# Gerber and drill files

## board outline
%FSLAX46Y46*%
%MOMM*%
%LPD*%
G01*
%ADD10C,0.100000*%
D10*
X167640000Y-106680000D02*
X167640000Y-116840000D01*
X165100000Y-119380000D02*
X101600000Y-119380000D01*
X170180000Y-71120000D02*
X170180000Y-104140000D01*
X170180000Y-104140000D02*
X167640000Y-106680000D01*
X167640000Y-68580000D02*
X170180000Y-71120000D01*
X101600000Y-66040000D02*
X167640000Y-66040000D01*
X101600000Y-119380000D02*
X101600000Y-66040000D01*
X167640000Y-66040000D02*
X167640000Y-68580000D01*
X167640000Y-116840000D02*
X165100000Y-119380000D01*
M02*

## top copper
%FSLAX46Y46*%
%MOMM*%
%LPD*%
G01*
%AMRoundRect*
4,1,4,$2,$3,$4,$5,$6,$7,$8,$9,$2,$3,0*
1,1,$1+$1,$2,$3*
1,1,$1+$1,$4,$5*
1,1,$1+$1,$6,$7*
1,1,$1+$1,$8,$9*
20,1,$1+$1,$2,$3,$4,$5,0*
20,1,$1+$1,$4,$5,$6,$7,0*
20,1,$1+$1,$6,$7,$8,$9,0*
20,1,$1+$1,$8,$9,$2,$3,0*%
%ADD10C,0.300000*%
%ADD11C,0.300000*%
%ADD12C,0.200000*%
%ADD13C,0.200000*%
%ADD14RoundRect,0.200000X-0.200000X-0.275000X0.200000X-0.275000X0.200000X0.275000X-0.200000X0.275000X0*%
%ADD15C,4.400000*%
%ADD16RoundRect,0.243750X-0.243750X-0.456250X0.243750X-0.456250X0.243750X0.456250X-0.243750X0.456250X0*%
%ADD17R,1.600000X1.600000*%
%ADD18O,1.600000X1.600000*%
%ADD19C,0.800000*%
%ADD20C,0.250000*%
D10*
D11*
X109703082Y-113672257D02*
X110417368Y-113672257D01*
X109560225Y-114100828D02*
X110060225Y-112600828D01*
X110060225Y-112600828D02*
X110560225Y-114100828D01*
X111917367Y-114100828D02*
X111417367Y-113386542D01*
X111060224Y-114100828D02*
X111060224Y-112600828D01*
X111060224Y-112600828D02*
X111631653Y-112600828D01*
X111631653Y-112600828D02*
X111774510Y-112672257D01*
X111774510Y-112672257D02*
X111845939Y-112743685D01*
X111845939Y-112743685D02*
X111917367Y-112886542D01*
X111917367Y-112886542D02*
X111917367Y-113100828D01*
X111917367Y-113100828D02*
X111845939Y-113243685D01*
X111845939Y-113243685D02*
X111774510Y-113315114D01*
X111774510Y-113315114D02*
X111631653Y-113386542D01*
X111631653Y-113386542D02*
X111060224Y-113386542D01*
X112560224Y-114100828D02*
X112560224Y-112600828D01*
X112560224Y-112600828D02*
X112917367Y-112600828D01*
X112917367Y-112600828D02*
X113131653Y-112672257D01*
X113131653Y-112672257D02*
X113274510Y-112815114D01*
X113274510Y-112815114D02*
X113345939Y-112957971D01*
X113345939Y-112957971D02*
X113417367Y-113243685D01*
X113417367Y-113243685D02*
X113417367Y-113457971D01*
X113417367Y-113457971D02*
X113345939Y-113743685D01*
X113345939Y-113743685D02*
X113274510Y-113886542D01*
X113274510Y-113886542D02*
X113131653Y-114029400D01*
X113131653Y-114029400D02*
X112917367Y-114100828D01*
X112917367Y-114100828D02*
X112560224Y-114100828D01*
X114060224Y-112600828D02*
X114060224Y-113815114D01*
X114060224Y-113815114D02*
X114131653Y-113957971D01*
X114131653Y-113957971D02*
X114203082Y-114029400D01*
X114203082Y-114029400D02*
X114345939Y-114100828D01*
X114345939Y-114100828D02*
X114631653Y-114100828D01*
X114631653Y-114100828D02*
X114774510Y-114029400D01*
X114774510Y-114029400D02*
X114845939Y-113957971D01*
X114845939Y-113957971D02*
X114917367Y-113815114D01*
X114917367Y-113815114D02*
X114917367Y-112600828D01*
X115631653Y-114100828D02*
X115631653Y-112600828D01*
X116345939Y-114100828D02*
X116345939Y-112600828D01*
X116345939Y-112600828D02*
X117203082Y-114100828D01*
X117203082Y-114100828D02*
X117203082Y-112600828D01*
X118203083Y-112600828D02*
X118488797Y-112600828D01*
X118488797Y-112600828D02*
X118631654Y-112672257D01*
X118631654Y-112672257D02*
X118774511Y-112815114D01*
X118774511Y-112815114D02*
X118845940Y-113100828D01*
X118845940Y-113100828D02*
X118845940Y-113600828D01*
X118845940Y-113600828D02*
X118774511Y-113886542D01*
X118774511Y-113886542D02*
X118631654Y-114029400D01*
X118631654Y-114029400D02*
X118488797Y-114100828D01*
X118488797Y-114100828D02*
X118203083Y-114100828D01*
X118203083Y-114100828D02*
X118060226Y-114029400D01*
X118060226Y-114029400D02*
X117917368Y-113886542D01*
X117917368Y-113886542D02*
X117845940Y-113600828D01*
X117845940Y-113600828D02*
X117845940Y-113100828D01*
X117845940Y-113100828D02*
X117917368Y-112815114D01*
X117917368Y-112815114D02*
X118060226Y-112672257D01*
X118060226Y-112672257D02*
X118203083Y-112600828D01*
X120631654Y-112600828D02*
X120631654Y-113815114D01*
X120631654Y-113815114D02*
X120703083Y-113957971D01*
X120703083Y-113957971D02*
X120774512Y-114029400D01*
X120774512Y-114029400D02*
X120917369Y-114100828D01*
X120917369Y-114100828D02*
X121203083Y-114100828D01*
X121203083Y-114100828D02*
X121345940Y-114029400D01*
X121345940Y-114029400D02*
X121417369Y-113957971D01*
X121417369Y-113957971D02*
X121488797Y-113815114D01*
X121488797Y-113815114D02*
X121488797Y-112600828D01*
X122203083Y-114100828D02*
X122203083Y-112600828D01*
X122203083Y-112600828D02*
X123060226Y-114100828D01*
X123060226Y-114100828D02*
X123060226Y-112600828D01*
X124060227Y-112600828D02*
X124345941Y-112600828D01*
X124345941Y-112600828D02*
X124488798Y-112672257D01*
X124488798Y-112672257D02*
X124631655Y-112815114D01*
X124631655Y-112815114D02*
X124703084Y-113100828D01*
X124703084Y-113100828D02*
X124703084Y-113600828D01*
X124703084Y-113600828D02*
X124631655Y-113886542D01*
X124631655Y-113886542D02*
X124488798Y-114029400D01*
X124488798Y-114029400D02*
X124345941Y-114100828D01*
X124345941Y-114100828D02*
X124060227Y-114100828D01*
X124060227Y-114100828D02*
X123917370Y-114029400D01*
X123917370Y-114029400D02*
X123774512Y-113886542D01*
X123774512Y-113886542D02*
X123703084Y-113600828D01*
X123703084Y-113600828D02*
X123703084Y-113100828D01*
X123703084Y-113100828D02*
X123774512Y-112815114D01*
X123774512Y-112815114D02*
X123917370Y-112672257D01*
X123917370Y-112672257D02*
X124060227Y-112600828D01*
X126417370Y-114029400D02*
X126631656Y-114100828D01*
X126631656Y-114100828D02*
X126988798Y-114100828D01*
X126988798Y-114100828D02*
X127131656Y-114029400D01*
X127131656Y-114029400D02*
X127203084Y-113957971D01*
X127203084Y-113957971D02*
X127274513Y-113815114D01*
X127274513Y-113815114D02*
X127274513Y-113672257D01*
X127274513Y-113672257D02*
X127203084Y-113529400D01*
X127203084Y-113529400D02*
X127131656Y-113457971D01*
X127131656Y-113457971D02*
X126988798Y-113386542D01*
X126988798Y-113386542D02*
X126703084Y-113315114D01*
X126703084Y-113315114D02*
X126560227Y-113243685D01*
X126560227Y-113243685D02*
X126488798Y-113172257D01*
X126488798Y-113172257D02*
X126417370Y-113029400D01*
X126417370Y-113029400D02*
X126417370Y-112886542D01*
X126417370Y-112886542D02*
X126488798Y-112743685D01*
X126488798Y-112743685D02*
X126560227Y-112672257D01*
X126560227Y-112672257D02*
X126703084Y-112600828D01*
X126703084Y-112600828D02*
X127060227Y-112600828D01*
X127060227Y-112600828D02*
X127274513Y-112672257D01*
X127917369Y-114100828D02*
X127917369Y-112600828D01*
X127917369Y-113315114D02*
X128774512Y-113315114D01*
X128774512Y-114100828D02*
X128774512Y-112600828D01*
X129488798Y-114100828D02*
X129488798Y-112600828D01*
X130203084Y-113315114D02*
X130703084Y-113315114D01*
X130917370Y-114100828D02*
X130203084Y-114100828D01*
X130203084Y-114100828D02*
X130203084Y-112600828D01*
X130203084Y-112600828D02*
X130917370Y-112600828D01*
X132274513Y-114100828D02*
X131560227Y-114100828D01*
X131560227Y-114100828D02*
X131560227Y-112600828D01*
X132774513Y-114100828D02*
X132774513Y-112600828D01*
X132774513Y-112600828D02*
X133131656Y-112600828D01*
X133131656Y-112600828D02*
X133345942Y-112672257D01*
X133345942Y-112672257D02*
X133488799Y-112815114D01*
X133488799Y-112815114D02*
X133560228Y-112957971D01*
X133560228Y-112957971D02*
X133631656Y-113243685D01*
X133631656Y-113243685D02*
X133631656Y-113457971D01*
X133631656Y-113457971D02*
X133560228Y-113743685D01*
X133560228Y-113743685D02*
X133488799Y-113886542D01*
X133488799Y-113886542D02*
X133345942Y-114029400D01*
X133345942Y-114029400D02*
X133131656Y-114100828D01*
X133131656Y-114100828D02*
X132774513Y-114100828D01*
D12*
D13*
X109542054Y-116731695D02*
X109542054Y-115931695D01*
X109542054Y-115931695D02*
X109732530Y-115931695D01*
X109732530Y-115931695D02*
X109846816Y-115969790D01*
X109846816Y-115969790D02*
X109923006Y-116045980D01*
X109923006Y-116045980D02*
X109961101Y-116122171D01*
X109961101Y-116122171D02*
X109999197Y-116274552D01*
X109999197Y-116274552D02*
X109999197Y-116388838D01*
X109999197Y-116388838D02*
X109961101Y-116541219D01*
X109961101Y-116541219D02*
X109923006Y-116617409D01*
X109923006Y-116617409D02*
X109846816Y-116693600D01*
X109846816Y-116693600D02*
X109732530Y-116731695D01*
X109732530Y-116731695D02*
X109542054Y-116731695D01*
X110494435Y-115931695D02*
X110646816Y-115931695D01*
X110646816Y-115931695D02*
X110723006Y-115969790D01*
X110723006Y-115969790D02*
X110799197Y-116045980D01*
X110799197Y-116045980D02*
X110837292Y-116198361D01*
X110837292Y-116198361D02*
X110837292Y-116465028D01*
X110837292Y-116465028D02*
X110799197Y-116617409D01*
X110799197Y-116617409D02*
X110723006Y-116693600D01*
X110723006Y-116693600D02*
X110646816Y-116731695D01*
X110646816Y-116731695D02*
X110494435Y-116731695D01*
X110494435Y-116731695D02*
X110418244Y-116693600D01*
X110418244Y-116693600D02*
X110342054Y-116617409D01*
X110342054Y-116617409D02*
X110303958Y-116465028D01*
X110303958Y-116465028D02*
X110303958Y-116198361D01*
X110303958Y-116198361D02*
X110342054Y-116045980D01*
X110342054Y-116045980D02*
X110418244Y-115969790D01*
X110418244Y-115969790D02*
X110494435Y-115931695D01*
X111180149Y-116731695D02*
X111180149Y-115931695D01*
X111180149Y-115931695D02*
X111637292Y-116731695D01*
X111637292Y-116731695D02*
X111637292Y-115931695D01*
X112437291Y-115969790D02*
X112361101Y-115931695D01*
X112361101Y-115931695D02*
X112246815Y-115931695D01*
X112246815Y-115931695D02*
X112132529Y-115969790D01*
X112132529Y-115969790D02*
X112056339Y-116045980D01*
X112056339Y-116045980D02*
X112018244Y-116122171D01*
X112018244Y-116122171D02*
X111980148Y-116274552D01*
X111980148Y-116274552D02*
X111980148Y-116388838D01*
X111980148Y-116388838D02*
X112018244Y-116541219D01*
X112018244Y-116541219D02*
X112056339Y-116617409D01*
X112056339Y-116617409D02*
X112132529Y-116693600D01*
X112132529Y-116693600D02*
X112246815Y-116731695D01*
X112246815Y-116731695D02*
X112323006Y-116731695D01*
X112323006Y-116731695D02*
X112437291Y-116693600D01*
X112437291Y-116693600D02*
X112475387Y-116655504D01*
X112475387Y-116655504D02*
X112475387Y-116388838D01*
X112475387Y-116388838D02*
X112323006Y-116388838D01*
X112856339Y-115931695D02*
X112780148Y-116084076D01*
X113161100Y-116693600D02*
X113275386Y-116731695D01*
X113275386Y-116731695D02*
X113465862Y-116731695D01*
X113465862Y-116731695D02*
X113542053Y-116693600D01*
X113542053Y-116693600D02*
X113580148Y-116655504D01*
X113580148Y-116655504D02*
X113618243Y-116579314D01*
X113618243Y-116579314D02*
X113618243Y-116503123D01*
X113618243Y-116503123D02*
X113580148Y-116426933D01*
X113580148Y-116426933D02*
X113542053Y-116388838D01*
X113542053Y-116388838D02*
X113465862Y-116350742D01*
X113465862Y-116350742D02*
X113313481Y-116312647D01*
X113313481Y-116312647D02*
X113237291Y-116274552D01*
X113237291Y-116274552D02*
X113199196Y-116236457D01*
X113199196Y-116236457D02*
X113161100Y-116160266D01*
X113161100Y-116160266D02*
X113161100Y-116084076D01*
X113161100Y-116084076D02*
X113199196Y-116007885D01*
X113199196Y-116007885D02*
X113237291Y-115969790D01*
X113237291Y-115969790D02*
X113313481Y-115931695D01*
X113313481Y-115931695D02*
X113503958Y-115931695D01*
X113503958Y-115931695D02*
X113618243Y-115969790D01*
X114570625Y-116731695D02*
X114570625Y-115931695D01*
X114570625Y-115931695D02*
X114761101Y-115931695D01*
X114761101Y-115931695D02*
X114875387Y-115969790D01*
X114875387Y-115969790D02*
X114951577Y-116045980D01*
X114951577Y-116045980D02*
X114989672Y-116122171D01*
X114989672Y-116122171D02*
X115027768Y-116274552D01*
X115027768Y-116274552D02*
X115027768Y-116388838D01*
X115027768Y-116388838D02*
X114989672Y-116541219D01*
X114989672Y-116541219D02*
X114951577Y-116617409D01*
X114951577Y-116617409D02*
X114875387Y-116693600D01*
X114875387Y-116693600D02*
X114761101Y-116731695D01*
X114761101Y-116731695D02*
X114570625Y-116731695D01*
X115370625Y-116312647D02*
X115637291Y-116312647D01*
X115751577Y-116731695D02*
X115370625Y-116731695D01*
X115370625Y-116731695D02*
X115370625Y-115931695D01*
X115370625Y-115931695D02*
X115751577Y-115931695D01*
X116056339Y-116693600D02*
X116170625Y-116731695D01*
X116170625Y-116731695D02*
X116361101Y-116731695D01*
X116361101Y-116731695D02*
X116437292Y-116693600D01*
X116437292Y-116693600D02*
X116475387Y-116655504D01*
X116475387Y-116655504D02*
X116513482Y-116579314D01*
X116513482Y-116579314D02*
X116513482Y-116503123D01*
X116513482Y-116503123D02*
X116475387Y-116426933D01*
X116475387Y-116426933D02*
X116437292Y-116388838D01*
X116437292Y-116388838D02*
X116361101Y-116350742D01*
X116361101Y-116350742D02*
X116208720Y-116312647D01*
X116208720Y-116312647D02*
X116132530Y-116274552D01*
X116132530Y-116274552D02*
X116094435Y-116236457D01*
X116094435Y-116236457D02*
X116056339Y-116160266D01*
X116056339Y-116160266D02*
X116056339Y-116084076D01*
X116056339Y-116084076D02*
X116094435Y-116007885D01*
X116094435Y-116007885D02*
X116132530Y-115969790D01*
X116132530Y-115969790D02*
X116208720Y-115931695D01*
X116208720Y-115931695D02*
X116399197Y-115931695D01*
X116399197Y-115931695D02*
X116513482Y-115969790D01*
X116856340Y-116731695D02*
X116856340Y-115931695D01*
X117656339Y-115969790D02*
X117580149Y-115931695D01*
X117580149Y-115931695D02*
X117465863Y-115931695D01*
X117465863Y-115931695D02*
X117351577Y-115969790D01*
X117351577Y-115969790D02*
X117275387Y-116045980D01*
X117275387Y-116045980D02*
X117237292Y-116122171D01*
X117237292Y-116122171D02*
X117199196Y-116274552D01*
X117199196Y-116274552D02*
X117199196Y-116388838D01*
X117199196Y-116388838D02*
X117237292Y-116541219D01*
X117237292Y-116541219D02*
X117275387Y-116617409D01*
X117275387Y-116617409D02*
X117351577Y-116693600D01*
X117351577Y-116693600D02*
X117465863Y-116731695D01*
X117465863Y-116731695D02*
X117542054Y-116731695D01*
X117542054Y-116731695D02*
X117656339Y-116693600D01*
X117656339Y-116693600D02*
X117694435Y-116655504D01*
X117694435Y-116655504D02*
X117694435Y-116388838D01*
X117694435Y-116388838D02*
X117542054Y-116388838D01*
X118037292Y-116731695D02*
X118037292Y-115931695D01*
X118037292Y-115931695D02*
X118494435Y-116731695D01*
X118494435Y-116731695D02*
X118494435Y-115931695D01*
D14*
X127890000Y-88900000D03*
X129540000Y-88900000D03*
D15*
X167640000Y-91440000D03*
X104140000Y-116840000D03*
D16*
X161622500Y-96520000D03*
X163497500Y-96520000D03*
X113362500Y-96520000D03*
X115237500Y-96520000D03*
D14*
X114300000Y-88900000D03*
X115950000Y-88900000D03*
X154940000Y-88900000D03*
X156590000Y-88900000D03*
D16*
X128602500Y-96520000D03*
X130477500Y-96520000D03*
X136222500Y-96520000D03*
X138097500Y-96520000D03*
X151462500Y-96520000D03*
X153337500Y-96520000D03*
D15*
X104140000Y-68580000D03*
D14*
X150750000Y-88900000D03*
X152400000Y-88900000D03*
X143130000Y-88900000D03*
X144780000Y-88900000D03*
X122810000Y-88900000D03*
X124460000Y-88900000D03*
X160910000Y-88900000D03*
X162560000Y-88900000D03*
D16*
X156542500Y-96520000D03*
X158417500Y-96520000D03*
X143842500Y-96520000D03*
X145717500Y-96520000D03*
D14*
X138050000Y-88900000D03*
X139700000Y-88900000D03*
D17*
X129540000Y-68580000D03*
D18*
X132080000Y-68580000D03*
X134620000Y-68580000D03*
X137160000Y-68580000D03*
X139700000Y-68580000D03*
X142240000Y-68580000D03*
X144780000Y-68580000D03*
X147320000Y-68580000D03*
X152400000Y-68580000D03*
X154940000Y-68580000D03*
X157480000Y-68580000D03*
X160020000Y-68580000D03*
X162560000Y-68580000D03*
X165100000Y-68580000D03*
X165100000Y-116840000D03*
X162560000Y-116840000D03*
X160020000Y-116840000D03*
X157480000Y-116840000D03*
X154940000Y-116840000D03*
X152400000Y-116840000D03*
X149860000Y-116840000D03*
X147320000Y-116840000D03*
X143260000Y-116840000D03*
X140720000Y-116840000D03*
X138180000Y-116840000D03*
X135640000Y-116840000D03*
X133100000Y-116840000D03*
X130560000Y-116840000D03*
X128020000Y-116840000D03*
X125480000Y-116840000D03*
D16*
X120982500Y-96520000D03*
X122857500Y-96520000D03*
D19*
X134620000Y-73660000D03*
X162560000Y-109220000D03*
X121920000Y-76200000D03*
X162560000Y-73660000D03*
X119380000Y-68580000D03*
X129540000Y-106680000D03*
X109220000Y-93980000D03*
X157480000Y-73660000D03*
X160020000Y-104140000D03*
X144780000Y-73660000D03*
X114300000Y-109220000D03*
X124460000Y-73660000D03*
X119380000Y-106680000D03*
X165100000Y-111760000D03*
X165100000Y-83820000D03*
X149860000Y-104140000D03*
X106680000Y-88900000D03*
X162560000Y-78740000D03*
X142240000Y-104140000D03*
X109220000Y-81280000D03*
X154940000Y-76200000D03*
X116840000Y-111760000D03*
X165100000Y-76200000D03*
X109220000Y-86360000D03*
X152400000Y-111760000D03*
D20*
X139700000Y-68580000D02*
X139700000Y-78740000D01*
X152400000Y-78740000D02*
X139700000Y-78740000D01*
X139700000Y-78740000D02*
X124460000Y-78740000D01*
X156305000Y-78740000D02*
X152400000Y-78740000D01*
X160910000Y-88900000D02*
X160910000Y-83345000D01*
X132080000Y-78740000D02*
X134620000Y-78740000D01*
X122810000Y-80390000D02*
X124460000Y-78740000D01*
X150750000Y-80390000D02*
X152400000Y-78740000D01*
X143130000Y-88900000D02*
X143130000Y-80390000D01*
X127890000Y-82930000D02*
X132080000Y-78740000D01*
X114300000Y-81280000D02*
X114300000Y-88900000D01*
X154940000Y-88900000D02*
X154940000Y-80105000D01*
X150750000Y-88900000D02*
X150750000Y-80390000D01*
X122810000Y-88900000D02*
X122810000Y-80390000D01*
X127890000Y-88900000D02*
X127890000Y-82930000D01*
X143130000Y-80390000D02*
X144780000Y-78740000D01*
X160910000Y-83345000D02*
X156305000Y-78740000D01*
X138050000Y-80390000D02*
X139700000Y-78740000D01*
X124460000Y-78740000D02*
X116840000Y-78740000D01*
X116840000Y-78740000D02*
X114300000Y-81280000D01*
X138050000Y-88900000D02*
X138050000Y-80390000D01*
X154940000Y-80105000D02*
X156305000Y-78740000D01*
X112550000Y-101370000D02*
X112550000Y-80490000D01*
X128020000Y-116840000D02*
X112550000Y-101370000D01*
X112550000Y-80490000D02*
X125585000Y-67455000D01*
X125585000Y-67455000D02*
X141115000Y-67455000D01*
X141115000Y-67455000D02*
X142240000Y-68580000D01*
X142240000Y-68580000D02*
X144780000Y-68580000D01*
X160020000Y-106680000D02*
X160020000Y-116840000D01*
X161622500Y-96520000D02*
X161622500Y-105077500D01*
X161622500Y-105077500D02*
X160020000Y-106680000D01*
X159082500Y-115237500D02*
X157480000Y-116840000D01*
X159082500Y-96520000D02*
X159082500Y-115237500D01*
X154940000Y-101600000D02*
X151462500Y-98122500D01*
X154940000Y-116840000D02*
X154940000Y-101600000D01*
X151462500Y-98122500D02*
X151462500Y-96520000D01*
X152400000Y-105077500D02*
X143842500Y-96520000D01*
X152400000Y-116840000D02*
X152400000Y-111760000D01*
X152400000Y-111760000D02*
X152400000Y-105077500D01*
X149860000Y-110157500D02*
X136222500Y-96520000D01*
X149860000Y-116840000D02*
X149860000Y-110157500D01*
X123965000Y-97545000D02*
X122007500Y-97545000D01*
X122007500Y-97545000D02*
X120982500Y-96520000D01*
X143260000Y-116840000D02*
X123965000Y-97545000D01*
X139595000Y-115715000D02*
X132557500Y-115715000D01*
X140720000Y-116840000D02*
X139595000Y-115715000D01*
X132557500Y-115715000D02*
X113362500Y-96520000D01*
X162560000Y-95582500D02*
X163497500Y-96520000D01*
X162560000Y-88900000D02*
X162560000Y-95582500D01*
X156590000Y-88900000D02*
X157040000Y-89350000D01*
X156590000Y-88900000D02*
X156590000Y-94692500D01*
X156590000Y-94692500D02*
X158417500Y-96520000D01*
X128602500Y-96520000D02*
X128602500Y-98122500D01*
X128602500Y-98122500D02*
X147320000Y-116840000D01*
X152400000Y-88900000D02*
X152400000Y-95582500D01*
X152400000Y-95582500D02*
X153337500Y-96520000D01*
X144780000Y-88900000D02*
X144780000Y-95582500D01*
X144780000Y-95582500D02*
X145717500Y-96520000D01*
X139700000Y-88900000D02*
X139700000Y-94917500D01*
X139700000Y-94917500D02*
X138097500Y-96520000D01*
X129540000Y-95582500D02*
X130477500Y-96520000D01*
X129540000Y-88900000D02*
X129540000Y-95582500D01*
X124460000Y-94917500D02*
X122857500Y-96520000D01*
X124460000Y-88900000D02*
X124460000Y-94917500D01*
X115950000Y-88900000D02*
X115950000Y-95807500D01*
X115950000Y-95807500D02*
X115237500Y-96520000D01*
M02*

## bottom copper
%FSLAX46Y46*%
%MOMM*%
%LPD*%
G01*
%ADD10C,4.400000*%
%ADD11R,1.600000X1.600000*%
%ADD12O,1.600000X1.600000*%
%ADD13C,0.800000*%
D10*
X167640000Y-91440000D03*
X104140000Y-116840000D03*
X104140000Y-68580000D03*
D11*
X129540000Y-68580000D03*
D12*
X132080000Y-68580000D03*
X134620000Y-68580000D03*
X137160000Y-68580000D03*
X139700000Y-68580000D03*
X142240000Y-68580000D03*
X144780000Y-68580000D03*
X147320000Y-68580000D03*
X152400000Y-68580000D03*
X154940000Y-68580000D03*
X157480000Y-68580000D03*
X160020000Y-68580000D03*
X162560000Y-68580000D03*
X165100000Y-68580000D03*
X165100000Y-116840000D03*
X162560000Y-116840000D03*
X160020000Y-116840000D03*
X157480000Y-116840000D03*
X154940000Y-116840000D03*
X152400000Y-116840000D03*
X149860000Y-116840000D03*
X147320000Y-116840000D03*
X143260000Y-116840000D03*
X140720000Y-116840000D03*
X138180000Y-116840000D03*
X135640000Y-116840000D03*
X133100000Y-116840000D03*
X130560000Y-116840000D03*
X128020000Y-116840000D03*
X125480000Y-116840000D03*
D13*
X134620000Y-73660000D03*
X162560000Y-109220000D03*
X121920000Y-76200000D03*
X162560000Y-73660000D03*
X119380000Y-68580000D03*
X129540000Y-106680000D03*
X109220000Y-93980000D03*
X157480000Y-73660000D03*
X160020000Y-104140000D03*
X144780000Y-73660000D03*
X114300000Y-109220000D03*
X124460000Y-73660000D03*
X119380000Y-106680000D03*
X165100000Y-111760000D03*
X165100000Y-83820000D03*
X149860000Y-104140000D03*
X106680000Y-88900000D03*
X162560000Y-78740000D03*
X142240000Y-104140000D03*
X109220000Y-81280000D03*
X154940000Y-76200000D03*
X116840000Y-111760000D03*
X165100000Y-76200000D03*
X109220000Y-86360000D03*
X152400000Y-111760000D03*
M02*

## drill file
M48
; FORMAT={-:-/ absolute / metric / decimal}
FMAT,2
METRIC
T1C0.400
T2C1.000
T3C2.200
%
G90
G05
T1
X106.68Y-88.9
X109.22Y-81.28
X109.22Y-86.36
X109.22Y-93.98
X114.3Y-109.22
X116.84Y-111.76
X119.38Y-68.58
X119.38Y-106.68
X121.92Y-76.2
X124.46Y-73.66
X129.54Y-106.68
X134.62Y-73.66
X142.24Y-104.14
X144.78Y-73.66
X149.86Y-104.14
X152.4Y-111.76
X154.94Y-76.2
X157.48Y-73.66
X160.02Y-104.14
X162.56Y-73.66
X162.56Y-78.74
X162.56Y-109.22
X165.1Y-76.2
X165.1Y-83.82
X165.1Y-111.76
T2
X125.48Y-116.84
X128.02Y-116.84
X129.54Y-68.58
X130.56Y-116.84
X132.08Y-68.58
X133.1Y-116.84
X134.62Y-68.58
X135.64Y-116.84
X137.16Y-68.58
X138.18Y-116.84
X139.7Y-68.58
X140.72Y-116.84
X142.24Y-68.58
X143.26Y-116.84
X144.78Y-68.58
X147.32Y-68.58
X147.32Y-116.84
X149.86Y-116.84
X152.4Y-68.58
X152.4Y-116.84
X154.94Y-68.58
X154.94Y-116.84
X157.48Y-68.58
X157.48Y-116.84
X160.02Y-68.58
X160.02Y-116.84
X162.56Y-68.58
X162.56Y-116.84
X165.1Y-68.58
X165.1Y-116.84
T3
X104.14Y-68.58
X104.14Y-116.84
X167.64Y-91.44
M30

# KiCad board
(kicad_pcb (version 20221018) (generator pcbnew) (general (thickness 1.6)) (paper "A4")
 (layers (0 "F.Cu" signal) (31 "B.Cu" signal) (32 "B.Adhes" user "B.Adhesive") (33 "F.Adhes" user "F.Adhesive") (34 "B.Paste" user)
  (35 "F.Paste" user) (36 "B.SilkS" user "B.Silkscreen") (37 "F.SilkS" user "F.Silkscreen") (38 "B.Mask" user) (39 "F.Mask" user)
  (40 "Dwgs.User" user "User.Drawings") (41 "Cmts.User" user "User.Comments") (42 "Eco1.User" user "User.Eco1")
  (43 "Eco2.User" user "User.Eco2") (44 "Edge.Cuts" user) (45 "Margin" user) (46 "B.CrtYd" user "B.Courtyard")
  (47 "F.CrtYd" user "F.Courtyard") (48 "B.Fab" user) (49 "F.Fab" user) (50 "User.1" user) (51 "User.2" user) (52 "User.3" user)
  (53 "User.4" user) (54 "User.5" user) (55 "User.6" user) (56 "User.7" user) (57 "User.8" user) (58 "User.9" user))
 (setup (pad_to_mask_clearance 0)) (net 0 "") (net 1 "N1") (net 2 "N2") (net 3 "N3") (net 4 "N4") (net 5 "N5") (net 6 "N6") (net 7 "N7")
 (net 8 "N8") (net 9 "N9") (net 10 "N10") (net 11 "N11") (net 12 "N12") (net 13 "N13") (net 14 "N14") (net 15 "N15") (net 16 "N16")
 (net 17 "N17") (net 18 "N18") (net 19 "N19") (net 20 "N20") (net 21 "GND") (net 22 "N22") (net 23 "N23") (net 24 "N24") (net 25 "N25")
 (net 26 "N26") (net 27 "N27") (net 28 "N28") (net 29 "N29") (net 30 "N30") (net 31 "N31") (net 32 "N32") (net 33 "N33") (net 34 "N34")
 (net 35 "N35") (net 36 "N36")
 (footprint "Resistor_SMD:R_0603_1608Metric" (layer "F.Cu") (at 128.715 88.9)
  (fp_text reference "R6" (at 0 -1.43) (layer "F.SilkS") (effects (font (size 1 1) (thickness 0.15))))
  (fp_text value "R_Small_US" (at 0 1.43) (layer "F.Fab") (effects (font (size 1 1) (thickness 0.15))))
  (pad "1" smd roundrect (at -0.825 0) (size 0.8 0.95) (layers "F.Cu" "F.Paste" "F.Mask") (roundrect_rratio 0.25) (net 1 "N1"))
  (pad "2" smd roundrect (at 0.825 0) (size 0.8 0.95) (layers "F.Cu" "F.Paste" "F.Mask") (roundrect_rratio 0.25) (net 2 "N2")))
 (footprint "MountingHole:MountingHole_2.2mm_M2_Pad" (layer "F.Cu") (at 167.64 91.44)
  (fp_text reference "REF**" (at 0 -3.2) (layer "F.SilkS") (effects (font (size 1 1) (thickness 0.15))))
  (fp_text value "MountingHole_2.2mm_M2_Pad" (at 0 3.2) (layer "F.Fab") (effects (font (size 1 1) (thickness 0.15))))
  (pad "1" thru_hole circle (at 0 0) (size 4.4 4.4) (drill 2.2) (layers "*.Cu" "*.Mask")))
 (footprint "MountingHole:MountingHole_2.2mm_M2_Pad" (layer "F.Cu") (at 104.14 116.84)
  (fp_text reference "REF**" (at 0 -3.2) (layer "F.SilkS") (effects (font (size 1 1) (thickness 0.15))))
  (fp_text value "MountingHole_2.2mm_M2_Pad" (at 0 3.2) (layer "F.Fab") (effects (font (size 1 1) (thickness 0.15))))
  (pad "1" thru_hole circle (at 0 0) (size 4.4 4.4) (drill 2.2) (layers "*.Cu" "*.Mask")))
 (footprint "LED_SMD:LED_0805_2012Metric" (layer "F.Cu") (at 162.56 96.52)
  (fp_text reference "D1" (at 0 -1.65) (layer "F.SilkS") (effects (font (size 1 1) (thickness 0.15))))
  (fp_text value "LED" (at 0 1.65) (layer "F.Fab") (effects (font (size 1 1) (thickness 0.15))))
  (pad "1" smd roundrect (at -0.9375 0) (size 0.975 1.4) (layers "F.Cu" "F.Paste" "F.Mask") (roundrect_rratio 0.25) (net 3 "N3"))
  (pad "2" smd roundrect (at 0.9375 0) (size 0.975 1.4) (layers "F.Cu" "F.Paste" "F.Mask") (roundrect_rratio 0.25) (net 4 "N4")))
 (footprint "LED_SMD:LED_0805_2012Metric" (layer "F.Cu") (at 114.3 96.52)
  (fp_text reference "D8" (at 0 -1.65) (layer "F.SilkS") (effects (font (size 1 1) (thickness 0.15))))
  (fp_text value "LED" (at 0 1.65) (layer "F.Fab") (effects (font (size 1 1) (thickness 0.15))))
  (pad "1" smd roundrect (at -0.9375 0) (size 0.975 1.4) (layers "F.Cu" "F.Paste" "F.Mask") (roundrect_rratio 0.25) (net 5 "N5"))
  (pad "2" smd roundrect (at 0.9375 0) (size 0.975 1.4) (layers "F.Cu" "F.Paste" "F.Mask") (roundrect_rratio 0.25) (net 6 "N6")))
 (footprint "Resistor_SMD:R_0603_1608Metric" (layer "F.Cu") (at 115.125 88.9)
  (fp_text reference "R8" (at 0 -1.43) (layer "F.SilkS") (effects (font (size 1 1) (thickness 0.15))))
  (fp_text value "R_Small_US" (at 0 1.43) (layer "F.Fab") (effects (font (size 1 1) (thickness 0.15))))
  (pad "1" smd roundrect (at -0.825 0) (size 0.8 0.95) (layers "F.Cu" "F.Paste" "F.Mask") (roundrect_rratio 0.25) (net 1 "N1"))
  (pad "2" smd roundrect (at 0.825 0) (size 0.8 0.95) (layers "F.Cu" "F.Paste" "F.Mask") (roundrect_rratio 0.25) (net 6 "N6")))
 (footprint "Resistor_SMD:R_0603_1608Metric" (layer "F.Cu") (at 155.765 88.9)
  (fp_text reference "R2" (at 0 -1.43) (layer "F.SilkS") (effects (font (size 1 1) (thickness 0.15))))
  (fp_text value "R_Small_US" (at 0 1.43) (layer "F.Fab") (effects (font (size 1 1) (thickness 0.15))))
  (pad "1" smd roundrect (at -0.825 0) (size 0.8 0.95) (layers "F.Cu" "F.Paste" "F.Mask") (roundrect_rratio 0.25) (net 1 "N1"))
  (pad "2" smd roundrect (at 0.825 0) (size 0.8 0.95) (layers "F.Cu" "F.Paste" "F.Mask") (roundrect_rratio 0.25) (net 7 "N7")))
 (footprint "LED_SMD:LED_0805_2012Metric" (layer "F.Cu") (at 129.54 96.52)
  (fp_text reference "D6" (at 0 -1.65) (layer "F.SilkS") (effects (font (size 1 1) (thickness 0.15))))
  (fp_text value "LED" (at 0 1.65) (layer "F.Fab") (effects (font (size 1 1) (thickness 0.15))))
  (pad "1" smd roundrect (at -0.9375 0) (size 0.975 1.4) (layers "F.Cu" "F.Paste" "F.Mask") (roundrect_rratio 0.25) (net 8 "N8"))
  (pad "2" smd roundrect (at 0.9375 0) (size 0.975 1.4) (layers "F.Cu" "F.Paste" "F.Mask") (roundrect_rratio 0.25) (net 2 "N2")))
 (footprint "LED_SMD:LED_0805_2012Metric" (layer "F.Cu") (at 137.16 96.52)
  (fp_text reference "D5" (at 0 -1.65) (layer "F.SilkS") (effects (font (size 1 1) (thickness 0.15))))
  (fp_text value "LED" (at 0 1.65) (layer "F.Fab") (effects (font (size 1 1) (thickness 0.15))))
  (pad "1" smd roundrect (at -0.9375 0) (size 0.975 1.4) (layers "F.Cu" "F.Paste" "F.Mask") (roundrect_rratio 0.25) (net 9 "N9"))
  (pad "2" smd roundrect (at 0.9375 0) (size 0.975 1.4) (layers "F.Cu" "F.Paste" "F.Mask") (roundrect_rratio 0.25) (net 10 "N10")))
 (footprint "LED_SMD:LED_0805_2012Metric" (layer "F.Cu") (at 152.4 96.52)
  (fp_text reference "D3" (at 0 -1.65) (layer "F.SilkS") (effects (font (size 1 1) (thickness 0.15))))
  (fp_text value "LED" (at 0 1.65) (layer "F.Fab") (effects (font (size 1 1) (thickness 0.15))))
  (pad "1" smd roundrect (at -0.9375 0) (size 0.975 1.4) (layers "F.Cu" "F.Paste" "F.Mask") (roundrect_rratio 0.25) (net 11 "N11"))
  (pad "2" smd roundrect (at 0.9375 0) (size 0.975 1.4) (layers "F.Cu" "F.Paste" "F.Mask") (roundrect_rratio 0.25) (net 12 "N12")))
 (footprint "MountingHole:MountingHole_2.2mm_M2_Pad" (layer "F.Cu") (at 104.14 68.58)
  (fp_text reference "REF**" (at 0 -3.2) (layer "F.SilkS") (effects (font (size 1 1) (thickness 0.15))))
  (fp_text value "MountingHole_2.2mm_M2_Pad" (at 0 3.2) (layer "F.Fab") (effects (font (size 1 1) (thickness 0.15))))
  (pad "1" thru_hole circle (at 0 0) (size 4.4 4.4) (drill 2.2) (layers "*.Cu" "*.Mask")))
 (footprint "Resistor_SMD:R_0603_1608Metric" (layer "F.Cu") (at 151.575 88.9)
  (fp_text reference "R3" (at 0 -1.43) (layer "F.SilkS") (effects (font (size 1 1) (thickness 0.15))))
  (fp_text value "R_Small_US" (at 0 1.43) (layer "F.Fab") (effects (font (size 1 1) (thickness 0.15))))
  (pad "1" smd roundrect (at -0.825 0) (size 0.8 0.95) (layers "F.Cu" "F.Paste" "F.Mask") (roundrect_rratio 0.25) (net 1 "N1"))
  (pad "2" smd roundrect (at 0.825 0) (size 0.8 0.95) (layers "F.Cu" "F.Paste" "F.Mask") (roundrect_rratio 0.25) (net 12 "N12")))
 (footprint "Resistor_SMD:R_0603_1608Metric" (layer "F.Cu") (at 143.955 88.9)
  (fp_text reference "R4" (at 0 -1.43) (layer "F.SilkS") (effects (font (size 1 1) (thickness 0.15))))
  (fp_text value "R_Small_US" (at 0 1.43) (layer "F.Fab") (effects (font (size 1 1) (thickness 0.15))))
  (pad "1" smd roundrect (at -0.825 0) (size 0.8 0.95) (layers "F.Cu" "F.Paste" "F.Mask") (roundrect_rratio 0.25) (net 1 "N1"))
  (pad "2" smd roundrect (at 0.825 0) (size 0.8 0.95) (layers "F.Cu" "F.Paste" "F.Mask") (roundrect_rratio 0.25) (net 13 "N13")))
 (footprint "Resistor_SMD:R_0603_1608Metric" (layer "F.Cu") (at 123.635 88.9)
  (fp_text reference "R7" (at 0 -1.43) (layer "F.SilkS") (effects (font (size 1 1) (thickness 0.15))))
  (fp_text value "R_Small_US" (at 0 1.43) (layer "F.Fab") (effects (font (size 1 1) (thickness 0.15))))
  (pad "1" smd roundrect (at -0.825 0) (size 0.8 0.95) (layers "F.Cu" "F.Paste" "F.Mask") (roundrect_rratio 0.25) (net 1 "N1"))
  (pad "2" smd roundrect (at 0.825 0) (size 0.8 0.95) (layers "F.Cu" "F.Paste" "F.Mask") (roundrect_rratio 0.25) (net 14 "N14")))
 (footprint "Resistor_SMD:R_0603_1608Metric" (layer "F.Cu") (at 161.735 88.9)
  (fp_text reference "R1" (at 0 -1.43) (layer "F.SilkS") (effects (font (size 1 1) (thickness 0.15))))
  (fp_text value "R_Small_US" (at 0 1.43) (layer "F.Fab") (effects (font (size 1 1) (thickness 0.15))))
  (pad "1" smd roundrect (at -0.825 0) (size 0.8 0.95) (layers "F.Cu" "F.Paste" "F.Mask") (roundrect_rratio 0.25) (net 1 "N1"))
  (pad "2" smd roundrect (at 0.825 0) (size 0.8 0.95) (layers "F.Cu" "F.Paste" "F.Mask") (roundrect_rratio 0.25) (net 4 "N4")))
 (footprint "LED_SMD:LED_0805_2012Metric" (layer "F.Cu") (at 157.48 96.52)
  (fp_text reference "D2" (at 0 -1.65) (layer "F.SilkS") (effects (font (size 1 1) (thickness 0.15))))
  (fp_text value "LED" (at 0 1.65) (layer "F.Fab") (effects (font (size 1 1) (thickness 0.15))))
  (pad "1" smd roundrect (at -0.9375 0) (size 0.975 1.4) (layers "F.Cu" "F.Paste" "F.Mask") (roundrect_rratio 0.25) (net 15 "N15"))
  (pad "2" smd roundrect (at 0.9375 0) (size 0.975 1.4) (layers "F.Cu" "F.Paste" "F.Mask") (roundrect_rratio 0.25) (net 7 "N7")))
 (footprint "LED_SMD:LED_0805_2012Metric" (layer "F.Cu") (at 144.78 96.52)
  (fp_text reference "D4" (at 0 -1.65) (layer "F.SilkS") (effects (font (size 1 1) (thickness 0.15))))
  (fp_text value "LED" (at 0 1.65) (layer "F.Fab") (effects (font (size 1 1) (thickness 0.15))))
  (pad "1" smd roundrect (at -0.9375 0) (size 0.975 1.4) (layers "F.Cu" "F.Paste" "F.Mask") (roundrect_rratio 0.25) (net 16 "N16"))
  (pad "2" smd roundrect (at 0.9375 0) (size 0.975 1.4) (layers "F.Cu" "F.Paste" "F.Mask") (roundrect_rratio 0.25) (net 13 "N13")))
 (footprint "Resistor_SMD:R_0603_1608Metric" (layer "F.Cu") (at 138.875 88.9)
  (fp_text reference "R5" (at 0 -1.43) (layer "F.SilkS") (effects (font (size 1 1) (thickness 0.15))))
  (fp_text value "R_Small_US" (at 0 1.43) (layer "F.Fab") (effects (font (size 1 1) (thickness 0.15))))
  (pad "1" smd roundrect (at -0.825 0) (size 0.8 0.95) (layers "F.Cu" "F.Paste" "F.Mask") (roundrect_rratio 0.25) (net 1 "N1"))
  (pad "2" smd roundrect (at 0.825 0) (size 0.8 0.95) (layers "F.Cu" "F.Paste" "F.Mask") (roundrect_rratio 0.25) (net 10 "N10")))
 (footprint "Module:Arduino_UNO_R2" (layer "F.Cu") (at 129.54 68.58)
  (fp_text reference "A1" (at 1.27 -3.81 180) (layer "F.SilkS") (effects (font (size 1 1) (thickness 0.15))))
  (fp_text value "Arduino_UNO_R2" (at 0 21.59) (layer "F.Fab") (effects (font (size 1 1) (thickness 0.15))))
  (pad "1" thru_hole rect (at 0 0 90) (size 1.6 1.6) (drill 1) (layers "*.Cu" "*.Mask") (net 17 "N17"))
  (pad "2" thru_hole oval (at 2.54 0 90) (size 1.6 1.6) (drill 1) (layers "*.Cu" "*.Mask") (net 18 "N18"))
  (pad "3" thru_hole oval (at 5.08 0 90) (size 1.6 1.6) (drill 1) (layers "*.Cu" "*.Mask") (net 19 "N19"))
  (pad "4" thru_hole oval (at 7.62 0 90) (size 1.6 1.6) (drill 1) (layers "*.Cu" "*.Mask") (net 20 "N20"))
  (pad "5" thru_hole oval (at 10.16 0 90) (size 1.6 1.6) (drill 1) (layers "*.Cu" "*.Mask") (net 1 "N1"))
  (pad "6" thru_hole oval (at 12.7 0 90) (size 1.6 1.6) (drill 1) (layers "*.Cu" "*.Mask") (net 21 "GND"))
  (pad "7" thru_hole oval (at 15.24 0 90) (size 1.6 1.6) (drill 1) (layers "*.Cu" "*.Mask") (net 21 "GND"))
  (pad "8" thru_hole oval (at 17.78 0 90) (size 1.6 1.6) (drill 1) (layers "*.Cu" "*.Mask") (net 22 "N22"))
  (pad "9" thru_hole oval (at 22.86 0 90) (size 1.6 1.6) (drill 1) (layers "*.Cu" "*.Mask") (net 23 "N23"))
  (pad "10" thru_hole oval (at 25.4 0 90) (size 1.6 1.6) (drill 1) (layers "*.Cu" "*.Mask") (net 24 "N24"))
  (pad "11" thru_hole oval (at 27.94 0 90) (size 1.6 1.6) (drill 1) (layers "*.Cu" "*.Mask") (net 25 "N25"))
  (pad "12" thru_hole oval (at 30.48 0 90) (size 1.6 1.6) (drill 1) (layers "*.Cu" "*.Mask") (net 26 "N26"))
  (pad "13" thru_hole oval (at 33.02 0 90) (size 1.6 1.6) (drill 1) (layers "*.Cu" "*.Mask") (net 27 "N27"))
  (pad "14" thru_hole oval (at 35.56 0 90) (size 1.6 1.6) (drill 1) (layers "*.Cu" "*.Mask") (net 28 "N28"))
  (pad "15" thru_hole oval (at 35.56 48.26 90) (size 1.6 1.6) (drill 1) (layers "*.Cu" "*.Mask") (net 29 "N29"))
  (pad "16" thru_hole oval (at 33.02 48.26 90) (size 1.6 1.6) (drill 1) (layers "*.Cu" "*.Mask") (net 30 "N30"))
  (pad "17" thru_hole oval (at 30.48 48.26 90) (size 1.6 1.6) (drill 1) (layers "*.Cu" "*.Mask") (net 3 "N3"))
  (pad "18" thru_hole oval (at 27.94 48.26 90) (size 1.6 1.6) (drill 1) (layers "*.Cu" "*.Mask") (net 15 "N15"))
  (pad "19" thru_hole oval (at 25.4 48.26 90) (size 1.6 1.6) (drill 1) (layers "*.Cu" "*.Mask") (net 11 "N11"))
  (pad "20" thru_hole oval (at 22.86 48.26 90) (size 1.6 1.6) (drill 1) (layers "*.Cu" "*.Mask") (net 16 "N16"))
  (pad "21" thru_hole oval (at 20.32 48.26 90) (size 1.6 1.6) (drill 1) (layers "*.Cu" "*.Mask") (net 9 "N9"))
  (pad "22" thru_hole oval (at 17.78 48.26 90) (size 1.6 1.6) (drill 1) (layers "*.Cu" "*.Mask") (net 8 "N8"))
  (pad "23" thru_hole oval (at 13.72 48.26 90) (size 1.6 1.6) (drill 1) (layers "*.Cu" "*.Mask") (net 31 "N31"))
  (pad "24" thru_hole oval (at 11.18 48.26 90) (size 1.6 1.6) (drill 1) (layers "*.Cu" "*.Mask") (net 5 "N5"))
  (pad "25" thru_hole oval (at 8.64 48.26 90) (size 1.6 1.6) (drill 1) (layers "*.Cu" "*.Mask") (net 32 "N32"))
  (pad "26" thru_hole oval (at 6.1 48.26 90) (size 1.6 1.6) (drill 1) (layers "*.Cu" "*.Mask") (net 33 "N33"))
  (pad "27" thru_hole oval (at 3.56 48.26 90) (size 1.6 1.6) (drill 1) (layers "*.Cu" "*.Mask") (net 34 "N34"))
  (pad "28" thru_hole oval (at 1.02 48.26 90) (size 1.6 1.6) (drill 1) (layers "*.Cu" "*.Mask") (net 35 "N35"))
  (pad "29" thru_hole oval (at -1.52 48.26 90) (size 1.6 1.6) (drill 1) (layers "*.Cu" "*.Mask") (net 21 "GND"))
  (pad "30" thru_hole oval (at -4.06 48.26 90) (size 1.6 1.6) (drill 1) (layers "*.Cu" "*.Mask") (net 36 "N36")))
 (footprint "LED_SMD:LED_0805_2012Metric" (layer "F.Cu") (at 121.92 96.52)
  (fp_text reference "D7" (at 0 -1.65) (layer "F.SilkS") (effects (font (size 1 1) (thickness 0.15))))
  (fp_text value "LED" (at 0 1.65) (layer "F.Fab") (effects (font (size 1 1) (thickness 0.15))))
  (pad "1" smd roundrect (at -0.9375 0) (size 0.975 1.4) (layers "F.Cu" "F.Paste" "F.Mask") (roundrect_rratio 0.25) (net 31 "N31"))
  (pad "2" smd roundrect (at 0.9375 0) (size 0.975 1.4) (layers "F.Cu" "F.Paste" "F.Mask") (roundrect_rratio 0.25) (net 14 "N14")))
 (gr_line (start 167.64 106.68) (end 167.64 116.84) (stroke (width 0.1) (type default)) (layer "Edge.Cuts"))
 (gr_line (start 165.1 119.38) (end 101.6 119.38) (stroke (width 0.1) (type default)) (layer "Edge.Cuts"))
 (gr_line (start 170.18 71.12) (end 170.18 104.14) (stroke (width 0.1) (type default)) (layer "Edge.Cuts"))
 (gr_line (start 170.18 104.14) (end 167.64 106.68) (stroke (width 0.1) (type default)) (layer "Edge.Cuts"))
 (gr_line (start 167.64 68.58) (end 170.18 71.12) (stroke (width 0.1) (type default)) (layer "Edge.Cuts"))
 (gr_line (start 101.6 66.04) (end 167.64 66.04) (stroke (width 0.1) (type default)) (layer "Edge.Cuts"))
 (gr_line (start 101.6 119.38) (end 101.6 66.04) (stroke (width 0.1) (type default)) (layer "Edge.Cuts"))
 (gr_line (start 167.64 66.04) (end 167.64 68.58) (stroke (width 0.1) (type default)) (layer "Edge.Cuts"))
 (gr_line (start 167.64 116.84) (end 165.1 119.38) (stroke (width 0.1) (type default)) (layer "Edge.Cuts"))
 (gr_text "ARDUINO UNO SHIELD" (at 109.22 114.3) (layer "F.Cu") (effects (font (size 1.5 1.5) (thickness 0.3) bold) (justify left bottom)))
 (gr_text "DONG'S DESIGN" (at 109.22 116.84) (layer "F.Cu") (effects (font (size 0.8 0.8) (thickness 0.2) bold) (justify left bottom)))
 (via (at 134.62 73.66) (size 0.8) (drill 0.4) (layers "F.Cu" "B.Cu") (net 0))
 (via (at 162.56 109.22) (size 0.8) (drill 0.4) (layers "F.Cu" "B.Cu") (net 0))
 (via (at 121.92 76.2) (size 0.8) (drill 0.4) (layers "F.Cu" "B.Cu") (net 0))
 (via (at 162.56 73.66) (size 0.8) (drill 0.4) (layers "F.Cu" "B.Cu") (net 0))
 (via (at 119.38 68.58) (size 0.8) (drill 0.4) (layers "F.Cu" "B.Cu") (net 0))
 (via (at 129.54 106.68) (size 0.8) (drill 0.4) (layers "F.Cu" "B.Cu") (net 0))
 (via (at 109.22 93.98) (size 0.8) (drill 0.4) (layers "F.Cu" "B.Cu") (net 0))
 (via (at 157.48 73.66) (size 0.8) (drill 0.4) (layers "F.Cu" "B.Cu") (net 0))
 (via (at 160.02 104.14) (size 0.8) (drill 0.4) (layers "F.Cu" "B.Cu") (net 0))
 (via (at 144.78 73.66) (size 0.8) (drill 0.4) (layers "F.Cu" "B.Cu") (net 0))
 (via (at 114.3 109.22) (size 0.8) (drill 0.4) (layers "F.Cu" "B.Cu") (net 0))
 (via (at 124.46 73.66) (size 0.8) (drill 0.4) (layers "F.Cu" "B.Cu") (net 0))
 (via (at 119.38 106.68) (size 0.8) (drill 0.4) (layers "F.Cu" "B.Cu") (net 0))
 (via (at 165.1 111.76) (size 0.8) (drill 0.4) (layers "F.Cu" "B.Cu") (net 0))
 (via (at 165.1 83.82) (size 0.8) (drill 0.4) (layers "F.Cu" "B.Cu") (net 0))
 (via (at 149.86 104.14) (size 0.8) (drill 0.4) (layers "F.Cu" "B.Cu") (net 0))
 (via (at 106.68 88.9) (size 0.8) (drill 0.4) (layers "F.Cu" "B.Cu") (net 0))
 (via (at 162.56 78.74) (size 0.8) (drill 0.4) (layers "F.Cu" "B.Cu") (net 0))
 (via (at 142.24 104.14) (size 0.8) (drill 0.4) (layers "F.Cu" "B.Cu") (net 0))
 (via (at 109.22 81.28) (size 0.8) (drill 0.4) (layers "F.Cu" "B.Cu") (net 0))
 (via (at 154.94 76.2) (size 0.8) (drill 0.4) (layers "F.Cu" "B.Cu") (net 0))
 (via (at 116.84 111.76) (size 0.8) (drill 0.4) (layers "F.Cu" "B.Cu") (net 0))
 (via (at 165.1 76.2) (size 0.8) (drill 0.4) (layers "F.Cu" "B.Cu") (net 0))
 (via (at 109.22 86.36) (size 0.8) (drill 0.4) (layers "F.Cu" "B.Cu") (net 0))
 (segment (start 139.7 68.58) (end 139.7 78.74) (width 0.25) (layer "F.Cu") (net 1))
 (segment (start 152.4 78.74) (end 139.7 78.74) (width 0.25) (layer "F.Cu") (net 1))
 (segment (start 139.7 78.74) (end 124.46 78.74) (width 0.25) (layer "F.Cu") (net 1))
 (segment (start 156.305 78.74) (end 152.4 78.74) (width 0.25) (layer "F.Cu") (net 1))
 (segment (start 160.91 88.9) (end 160.91 83.345) (width 0.25) (layer "F.Cu") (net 1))
 (segment (start 132.08 78.74) (end 134.62 78.74) (width 0.25) (layer "F.Cu") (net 1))
 (segment (start 122.81 80.39) (end 124.46 78.74) (width 0.25) (layer "F.Cu") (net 1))
 (segment (start 150.75 80.39) (end 152.4 78.74) (width 0.25) (layer "F.Cu") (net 1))
 (segment (start 143.13 88.9) (end 143.13 80.39) (width 0.25) (layer "F.Cu") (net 1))
 (segment (start 127.89 82.93) (end 132.08 78.74) (width 0.25) (layer "F.Cu") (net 1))
 (segment (start 114.3 81.28) (end 114.3 88.9) (width 0.25) (layer "F.Cu") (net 1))
 (segment (start 154.94 88.9) (end 154.94 80.105) (width 0.25) (layer "F.Cu") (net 1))
 (segment (start 150.75 88.9) (end 150.75 80.39) (width 0.25) (layer "F.Cu") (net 1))
 (segment (start 122.81 88.9) (end 122.81 80.39) (width 0.25) (layer "F.Cu") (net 1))
 (segment (start 127.89 88.9) (end 127.89 82.93) (width 0.25) (layer "F.Cu") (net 1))
 (segment (start 143.13 80.39) (end 144.78 78.74) (width 0.25) (layer "F.Cu") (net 1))
 (segment (start 160.91 83.345) (end 156.305 78.74) (width 0.25) (layer "F.Cu") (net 1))
 (segment (start 138.05 80.39) (end 139.7 78.74) (width 0.25) (layer "F.Cu") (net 1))
 (segment (start 124.46 78.74) (end 116.84 78.74) (width 0.25) (layer "F.Cu") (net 1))
 (segment (start 116.84 78.74) (end 114.3 81.28) (width 0.25) (layer "F.Cu") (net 1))
 (segment (start 138.05 88.9) (end 138.05 80.39) (width 0.25) (layer "F.Cu") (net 1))
 (segment (start 154.94 80.105) (end 156.305 78.74) (width 0.25) (layer "F.Cu") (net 1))
 (segment (start 112.55 101.37) (end 112.55 80.49) (width 0.25) (layer "F.Cu") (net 21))
 (segment (start 128.02 116.84) (end 112.55 101.37) (width 0.25) (layer "F.Cu") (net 21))
 (segment (start 112.55 80.49) (end 125.585 67.455) (width 0.25) (layer "F.Cu") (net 21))
 (segment (start 125.585 67.455) (end 141.115 67.455) (width 0.25) (layer "F.Cu") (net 21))
 (segment (start 141.115 67.455) (end 142.24 68.58) (width 0.25) (layer "F.Cu") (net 21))
 (segment (start 142.24 68.58) (end 144.78 68.58) (width 0.25) (layer "F.Cu") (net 21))
 (segment (start 160.02 106.68) (end 160.02 116.84) (width 0.25) (layer "F.Cu") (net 3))
 (segment (start 161.6225 96.52) (end 161.6225 105.0775) (width 0.25) (layer "F.Cu") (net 3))
 (segment (start 161.6225 105.0775) (end 160.02 106.68) (width 0.25) (layer "F.Cu") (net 3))
 (segment (start 159.0825 115.2375) (end 157.48 116.84) (width 0.25) (layer "F.Cu") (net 15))
 (segment (start 159.0825 96.52) (end 159.0825 115.2375) (width 0.25) (layer "F.Cu") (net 15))
 (segment (start 154.94 101.6) (end 151.4625 98.1225) (width 0.25) (layer "F.Cu") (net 11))
 (segment (start 154.94 116.84) (end 154.94 101.6) (width 0.25) (layer "F.Cu") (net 11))
 (segment (start 151.4625 98.1225) (end 151.4625 96.52) (width 0.25) (layer "F.Cu") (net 11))
 (segment (start 152.4 105.0775) (end 143.8425 96.52) (width 0.25) (layer "F.Cu") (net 16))
 (segment (start 152.4 116.84) (end 152.4 111.76) (width 0.25) (layer "F.Cu") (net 16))
 (segment (start 152.4 111.76) (end 152.4 105.0775) (width 0.25) (layer "F.Cu") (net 16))
 (via (at 152.4 111.76) (size 0.8) (drill 0.4) (layers "F.Cu" "B.Cu") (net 16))
 (segment (start 149.86 110.1575) (end 136.2225 96.52) (width 0.25) (layer "F.Cu") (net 9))
 (segment (start 149.86 116.84) (end 149.86 110.1575) (width 0.25) (layer "F.Cu") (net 9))
 (segment (start 123.965 97.545) (end 122.0075 97.545) (width 0.25) (layer "F.Cu") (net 31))
 (segment (start 122.0075 97.545) (end 120.9825 96.52) (width 0.25) (layer "F.Cu") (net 31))
 (segment (start 143.26 116.84) (end 123.965 97.545) (width 0.25) (layer "F.Cu") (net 31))
 (segment (start 139.595 115.715) (end 132.5575 115.715) (width 0.25) (layer "F.Cu") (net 5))
 (segment (start 140.72 116.84) (end 139.595 115.715) (width 0.25) (layer "F.Cu") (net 5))
 (segment (start 132.5575 115.715) (end 113.3625 96.52) (width 0.25) (layer "F.Cu") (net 5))
 (segment (start 162.56 95.5825) (end 163.4975 96.52) (width 0.25) (layer "F.Cu") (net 4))
 (segment (start 162.56 88.9) (end 162.56 95.5825) (width 0.25) (layer "F.Cu") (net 4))
 (segment (start 156.59 88.9) (end 157.04 89.35) (width 0.25) (layer "F.Cu") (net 7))
 (segment (start 156.59 88.9) (end 156.59 94.6925) (width 0.25) (layer "F.Cu") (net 7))
 (segment (start 156.59 94.6925) (end 158.4175 96.52) (width 0.25) (layer "F.Cu") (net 7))
 (segment (start 128.6025 96.52) (end 128.6025 98.1225) (width 0.25) (layer "F.Cu") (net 8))
 (segment (start 128.6025 98.1225) (end 147.32 116.84) (width 0.25) (layer "F.Cu") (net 8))
 (segment (start 152.4 88.9) (end 152.4 95.5825) (width 0.25) (layer "F.Cu") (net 12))
 (segment (start 152.4 95.5825) (end 153.3375 96.52) (width 0.25) (layer "F.Cu") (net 12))
 (segment (start 144.78 88.9) (end 144.78 95.5825) (width 0.25) (layer "F.Cu") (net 13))
 (segment (start 144.78 95.5825) (end 145.7175 96.52) (width 0.25) (layer "F.Cu") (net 13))
 (segment (start 139.7 88.9) (end 139.7 94.9175) (width 0.25) (layer "F.Cu") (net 10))
 (segment (start 139.7 94.9175) (end 138.0975 96.52) (width 0.25) (layer "F.Cu") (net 10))
 (segment (start 129.54 95.5825) (end 130.4775 96.52) (width 0.25) (layer "F.Cu") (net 2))
 (segment (start 129.54 88.9) (end 129.54 95.5825) (width 0.25) (layer "F.Cu") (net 2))
 (segment (start 124.46 94.9175) (end 122.8575 96.52) (width 0.25) (layer "F.Cu") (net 14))
 (segment (start 124.46 88.9) (end 124.46 94.9175) (width 0.25) (layer "F.Cu") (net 14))
 (segment (start 115.95 88.9) (end 115.95 95.8075) (width 0.25) (layer "F.Cu") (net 6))
 (segment (start 115.95 95.8075) (end 115.2375 96.52) (width 0.25) (layer "F.Cu") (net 6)))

